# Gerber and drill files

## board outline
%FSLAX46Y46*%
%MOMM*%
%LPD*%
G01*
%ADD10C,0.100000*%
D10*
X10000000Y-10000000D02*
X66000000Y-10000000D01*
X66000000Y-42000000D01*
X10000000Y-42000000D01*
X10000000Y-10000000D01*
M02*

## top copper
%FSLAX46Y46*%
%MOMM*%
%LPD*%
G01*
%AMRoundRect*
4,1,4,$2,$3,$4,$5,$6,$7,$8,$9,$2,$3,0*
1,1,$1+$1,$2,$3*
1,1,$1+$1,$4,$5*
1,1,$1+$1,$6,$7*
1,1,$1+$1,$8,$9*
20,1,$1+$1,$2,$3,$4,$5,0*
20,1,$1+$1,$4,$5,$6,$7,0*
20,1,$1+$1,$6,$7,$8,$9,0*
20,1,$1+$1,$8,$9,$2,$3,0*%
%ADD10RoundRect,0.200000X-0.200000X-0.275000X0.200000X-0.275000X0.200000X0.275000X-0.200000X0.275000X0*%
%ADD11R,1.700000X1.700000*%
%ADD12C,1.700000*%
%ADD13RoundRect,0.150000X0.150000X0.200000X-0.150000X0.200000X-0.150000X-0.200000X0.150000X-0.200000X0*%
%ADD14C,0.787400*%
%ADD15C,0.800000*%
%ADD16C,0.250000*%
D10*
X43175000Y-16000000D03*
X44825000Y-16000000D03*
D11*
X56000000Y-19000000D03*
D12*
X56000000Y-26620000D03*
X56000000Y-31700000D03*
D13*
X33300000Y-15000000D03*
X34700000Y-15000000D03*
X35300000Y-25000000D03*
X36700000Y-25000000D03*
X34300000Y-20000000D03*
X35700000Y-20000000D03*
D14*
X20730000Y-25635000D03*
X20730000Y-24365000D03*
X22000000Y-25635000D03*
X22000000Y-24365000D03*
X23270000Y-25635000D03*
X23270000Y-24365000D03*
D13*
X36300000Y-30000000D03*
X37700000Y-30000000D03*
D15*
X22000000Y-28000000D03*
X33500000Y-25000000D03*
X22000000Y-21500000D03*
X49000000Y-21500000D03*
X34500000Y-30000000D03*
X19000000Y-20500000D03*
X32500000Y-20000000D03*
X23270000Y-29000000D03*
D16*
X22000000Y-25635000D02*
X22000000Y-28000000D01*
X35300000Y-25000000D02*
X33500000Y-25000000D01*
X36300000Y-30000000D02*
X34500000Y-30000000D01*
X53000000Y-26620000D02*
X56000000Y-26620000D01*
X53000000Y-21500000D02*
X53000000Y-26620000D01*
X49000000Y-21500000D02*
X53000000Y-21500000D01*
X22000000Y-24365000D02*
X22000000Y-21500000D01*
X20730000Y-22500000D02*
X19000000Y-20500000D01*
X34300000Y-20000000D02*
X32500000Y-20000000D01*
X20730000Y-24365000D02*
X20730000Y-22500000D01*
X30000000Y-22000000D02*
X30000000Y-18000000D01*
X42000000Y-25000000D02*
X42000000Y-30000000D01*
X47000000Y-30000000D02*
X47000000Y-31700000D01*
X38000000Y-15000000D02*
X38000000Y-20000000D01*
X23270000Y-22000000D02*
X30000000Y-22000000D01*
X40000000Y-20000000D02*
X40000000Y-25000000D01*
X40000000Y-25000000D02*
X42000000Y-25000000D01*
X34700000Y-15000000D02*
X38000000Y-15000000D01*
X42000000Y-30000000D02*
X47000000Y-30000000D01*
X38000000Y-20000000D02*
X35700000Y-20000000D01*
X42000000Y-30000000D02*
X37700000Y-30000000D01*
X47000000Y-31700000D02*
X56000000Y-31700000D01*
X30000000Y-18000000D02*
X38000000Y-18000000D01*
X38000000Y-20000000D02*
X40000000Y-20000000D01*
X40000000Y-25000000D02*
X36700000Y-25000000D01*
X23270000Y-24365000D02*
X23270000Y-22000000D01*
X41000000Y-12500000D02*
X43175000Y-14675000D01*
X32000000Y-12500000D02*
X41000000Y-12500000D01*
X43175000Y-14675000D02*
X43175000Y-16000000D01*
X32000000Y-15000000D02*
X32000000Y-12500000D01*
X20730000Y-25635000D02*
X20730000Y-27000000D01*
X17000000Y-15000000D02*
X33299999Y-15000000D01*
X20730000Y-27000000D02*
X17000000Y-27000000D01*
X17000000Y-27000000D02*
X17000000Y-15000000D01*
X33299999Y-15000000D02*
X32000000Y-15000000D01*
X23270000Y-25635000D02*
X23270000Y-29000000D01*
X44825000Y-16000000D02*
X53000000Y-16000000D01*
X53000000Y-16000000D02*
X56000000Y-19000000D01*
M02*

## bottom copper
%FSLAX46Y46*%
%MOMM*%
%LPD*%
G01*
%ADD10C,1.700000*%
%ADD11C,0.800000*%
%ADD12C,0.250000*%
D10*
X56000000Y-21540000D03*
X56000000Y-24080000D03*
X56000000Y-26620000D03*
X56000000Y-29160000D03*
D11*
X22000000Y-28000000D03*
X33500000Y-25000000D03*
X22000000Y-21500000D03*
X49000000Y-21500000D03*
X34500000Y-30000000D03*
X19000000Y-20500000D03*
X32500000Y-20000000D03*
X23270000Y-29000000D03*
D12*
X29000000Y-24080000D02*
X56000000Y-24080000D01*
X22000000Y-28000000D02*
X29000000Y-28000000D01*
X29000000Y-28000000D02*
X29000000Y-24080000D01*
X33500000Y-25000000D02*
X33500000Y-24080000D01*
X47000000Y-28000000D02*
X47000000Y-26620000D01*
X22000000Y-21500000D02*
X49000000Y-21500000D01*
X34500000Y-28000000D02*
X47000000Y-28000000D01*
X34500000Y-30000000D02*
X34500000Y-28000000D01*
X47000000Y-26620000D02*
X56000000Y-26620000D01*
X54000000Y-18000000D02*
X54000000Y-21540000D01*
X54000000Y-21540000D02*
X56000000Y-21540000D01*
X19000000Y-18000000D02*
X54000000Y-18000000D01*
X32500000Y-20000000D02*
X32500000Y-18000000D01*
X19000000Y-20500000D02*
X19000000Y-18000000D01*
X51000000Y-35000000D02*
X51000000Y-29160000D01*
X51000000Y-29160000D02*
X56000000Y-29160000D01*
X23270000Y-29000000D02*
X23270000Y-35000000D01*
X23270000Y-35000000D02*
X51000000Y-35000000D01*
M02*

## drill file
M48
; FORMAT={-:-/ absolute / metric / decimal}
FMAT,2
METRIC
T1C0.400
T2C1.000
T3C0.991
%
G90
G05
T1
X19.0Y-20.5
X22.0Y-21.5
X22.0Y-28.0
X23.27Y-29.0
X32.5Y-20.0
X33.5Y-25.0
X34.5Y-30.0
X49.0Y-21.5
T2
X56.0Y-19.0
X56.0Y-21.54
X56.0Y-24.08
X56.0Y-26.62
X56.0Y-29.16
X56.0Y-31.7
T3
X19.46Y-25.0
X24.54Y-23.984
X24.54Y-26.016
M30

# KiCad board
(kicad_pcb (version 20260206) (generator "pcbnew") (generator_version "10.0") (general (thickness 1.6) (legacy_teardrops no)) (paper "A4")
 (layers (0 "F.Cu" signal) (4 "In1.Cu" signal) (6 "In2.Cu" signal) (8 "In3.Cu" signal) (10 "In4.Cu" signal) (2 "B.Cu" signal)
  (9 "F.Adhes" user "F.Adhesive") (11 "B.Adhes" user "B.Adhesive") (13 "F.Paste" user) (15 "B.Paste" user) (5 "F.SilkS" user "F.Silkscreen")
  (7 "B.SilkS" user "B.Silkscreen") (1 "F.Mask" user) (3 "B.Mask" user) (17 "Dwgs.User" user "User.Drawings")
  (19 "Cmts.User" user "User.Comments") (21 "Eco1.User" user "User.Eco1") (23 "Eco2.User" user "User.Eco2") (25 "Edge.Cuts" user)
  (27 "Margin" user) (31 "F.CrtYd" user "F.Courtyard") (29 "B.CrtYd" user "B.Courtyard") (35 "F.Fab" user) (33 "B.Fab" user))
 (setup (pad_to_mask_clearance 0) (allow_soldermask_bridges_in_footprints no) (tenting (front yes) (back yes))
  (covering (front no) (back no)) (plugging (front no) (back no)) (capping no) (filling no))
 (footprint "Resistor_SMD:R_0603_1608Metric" (layer "F.Cu") (at 44 16)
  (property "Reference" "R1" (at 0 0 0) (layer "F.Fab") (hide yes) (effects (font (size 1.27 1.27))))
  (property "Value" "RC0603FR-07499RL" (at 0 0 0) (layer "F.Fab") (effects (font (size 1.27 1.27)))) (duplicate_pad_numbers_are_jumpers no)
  (pad "1" smd roundrect (at -0.825 0) (size 0.8 0.95) (layers "F.Cu" "F.Mask" "F.Paste") (roundrect_rratio 0.25) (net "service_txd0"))
  (pad "2" smd roundrect (at 0.825 0) (size 0.8 0.95) (layers "F.Cu" "F.Mask" "F.Paste") (roundrect_rratio 0.25) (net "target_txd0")))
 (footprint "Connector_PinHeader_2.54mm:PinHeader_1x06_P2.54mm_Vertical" (layer "F.Cu") (at 56 19)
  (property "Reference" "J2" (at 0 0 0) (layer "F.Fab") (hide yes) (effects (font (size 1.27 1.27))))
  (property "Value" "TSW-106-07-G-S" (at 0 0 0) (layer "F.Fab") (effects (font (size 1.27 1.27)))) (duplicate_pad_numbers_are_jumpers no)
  (pad "1" thru_hole rect (at 0 0) (size 1.7 1.7) (drill 1) (layers "*.Cu" "*.Mask") (remove_unused_layers yes) (keep_end_layers no)
   (zone_layer_connections) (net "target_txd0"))
  (pad "2" thru_hole circle (at 0 2.54) (size 1.7 1.7) (drill 1) (layers "*.Cu" "*.Mask") (remove_unused_layers yes) (keep_end_layers no)
   (zone_layer_connections) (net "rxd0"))
  (pad "3" thru_hole circle (at 0 5.08) (size 1.7 1.7) (drill 1) (layers "*.Cu" "*.Mask") (remove_unused_layers yes) (keep_end_layers no)
   (zone_layer_connections) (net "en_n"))
  (pad "4" thru_hole circle (at 0 7.62) (size 1.7 1.7) (drill 1) (layers "*.Cu" "*.Mask") (remove_unused_layers yes) (keep_end_layers no)
   (zone_layer_connections) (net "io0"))
  (pad "5" thru_hole circle (at 0 10.16) (size 1.7 1.7) (drill 1) (layers "*.Cu" "*.Mask") (remove_unused_layers yes) (keep_end_layers no)
   (zone_layer_connections) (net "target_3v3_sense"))
  (pad "6" thru_hole circle (at 0 12.7) (size 1.7 1.7) (drill 1) (layers "*.Cu" "*.Mask") (remove_unused_layers yes) (keep_end_layers no)
   (zone_layer_connections) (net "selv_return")))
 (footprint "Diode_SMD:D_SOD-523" (layer "F.Cu") (at 34 15)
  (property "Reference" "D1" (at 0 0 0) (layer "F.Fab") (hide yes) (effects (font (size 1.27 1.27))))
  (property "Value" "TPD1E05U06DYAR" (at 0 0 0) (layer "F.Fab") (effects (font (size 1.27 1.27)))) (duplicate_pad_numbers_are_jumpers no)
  (pad "1" smd roundrect (at -0.7 0 180) (size 0.6 0.7) (layers "F.Cu" "F.Mask" "F.Paste") (roundrect_rratio 0.25) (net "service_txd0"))
  (pad "2" smd roundrect (at 0.7 0 180) (size 0.6 0.7) (layers "F.Cu" "F.Mask" "F.Paste") (roundrect_rratio 0.25) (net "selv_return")))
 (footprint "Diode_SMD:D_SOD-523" (layer "F.Cu") (at 36 25)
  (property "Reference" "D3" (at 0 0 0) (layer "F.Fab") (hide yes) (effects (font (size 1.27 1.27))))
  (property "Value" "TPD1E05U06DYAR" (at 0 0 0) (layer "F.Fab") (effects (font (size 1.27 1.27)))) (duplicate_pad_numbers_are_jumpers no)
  (pad "1" smd roundrect (at -0.7 0 180) (size 0.6 0.7) (layers "F.Cu" "F.Mask" "F.Paste") (roundrect_rratio 0.25) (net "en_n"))
  (pad "2" smd roundrect (at 0.7 0 180) (size 0.6 0.7) (layers "F.Cu" "F.Mask" "F.Paste") (roundrect_rratio 0.25) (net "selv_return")))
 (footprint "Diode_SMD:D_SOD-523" (layer "F.Cu") (at 35 20)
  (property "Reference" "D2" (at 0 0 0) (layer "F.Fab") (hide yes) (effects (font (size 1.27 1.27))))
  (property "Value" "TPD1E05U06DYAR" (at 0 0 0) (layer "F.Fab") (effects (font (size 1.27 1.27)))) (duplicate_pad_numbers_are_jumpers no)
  (pad "1" smd roundrect (at -0.7 0 180) (size 0.6 0.7) (layers "F.Cu" "F.Mask" "F.Paste") (roundrect_rratio 0.25) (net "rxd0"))
  (pad "2" smd roundrect (at 0.7 0 180) (size 0.6 0.7) (layers "F.Cu" "F.Mask" "F.Paste") (roundrect_rratio 0.25) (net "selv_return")))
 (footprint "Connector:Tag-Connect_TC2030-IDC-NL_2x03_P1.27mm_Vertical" (layer "F.Cu") (at 22 25)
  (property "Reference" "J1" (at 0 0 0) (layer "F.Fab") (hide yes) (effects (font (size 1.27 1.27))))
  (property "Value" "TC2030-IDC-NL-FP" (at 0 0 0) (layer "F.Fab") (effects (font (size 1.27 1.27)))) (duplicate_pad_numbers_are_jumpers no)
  (pad "" np_thru_hole circle (at -2.54 0) (size 0.9906 0.9906) (drill 0.9906) (layers "*.Cu" "*.Mask"))
  (pad "" np_thru_hole circle (at 2.54 -1.016) (size 0.9906 0.9906) (drill 0.9906) (layers "*.Cu" "*.Mask"))
  (pad "" np_thru_hole circle (at 2.54 1.016) (size 0.9906 0.9906) (drill 0.9906) (layers "*.Cu" "*.Mask"))
  (pad "1" connect circle (at -1.27 0.635) (size 0.7874 0.7874) (layers "F.Cu" "F.Mask") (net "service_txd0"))
  (pad "2" connect circle (at -1.27 -0.635) (size 0.7874 0.7874) (layers "F.Cu" "F.Mask") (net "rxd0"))
  (pad "3" connect circle (at 0 0.635) (size 0.7874 0.7874) (layers "F.Cu" "F.Mask") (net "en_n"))
  (pad "4" connect circle (at 0 -0.635) (size 0.7874 0.7874) (layers "F.Cu" "F.Mask") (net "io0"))
  (pad "5" connect circle (at 1.27 0.635) (size 0.7874 0.7874) (layers "F.Cu" "F.Mask") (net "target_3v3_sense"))
  (pad "6" connect circle (at 1.27 -0.635) (size 0.7874 0.7874) (layers "F.Cu" "F.Mask") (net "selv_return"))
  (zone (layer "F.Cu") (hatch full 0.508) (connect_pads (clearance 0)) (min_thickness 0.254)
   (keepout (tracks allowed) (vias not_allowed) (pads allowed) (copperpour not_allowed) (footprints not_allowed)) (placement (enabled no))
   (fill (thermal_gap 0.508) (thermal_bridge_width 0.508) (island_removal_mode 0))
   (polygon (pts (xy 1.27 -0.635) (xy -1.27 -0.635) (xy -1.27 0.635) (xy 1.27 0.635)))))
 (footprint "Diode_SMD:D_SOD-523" (layer "F.Cu") (at 37 30)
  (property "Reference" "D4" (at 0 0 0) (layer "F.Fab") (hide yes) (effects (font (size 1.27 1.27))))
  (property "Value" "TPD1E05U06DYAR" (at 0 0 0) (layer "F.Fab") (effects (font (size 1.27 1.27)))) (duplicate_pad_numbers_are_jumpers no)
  (pad "1" smd roundrect (at -0.7 0 180) (size 0.6 0.7) (layers "F.Cu" "F.Mask" "F.Paste") (roundrect_rratio 0.25) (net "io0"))
  (pad "2" smd roundrect (at 0.7 0 180) (size 0.6 0.7) (layers "F.Cu" "F.Mask" "F.Paste") (roundrect_rratio 0.25) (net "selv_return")))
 (gr_poly (pts (xy 10 10) (xy 66 10) (xy 66 42) (xy 10 42)) (stroke (width 0.1) (type solid)) (fill no) (layer "Edge.Cuts"))
 (segment (start 22 25.635) (end 22 28) (width 0.25) (layer "F.Cu") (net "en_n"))
 (segment (start 35.3 25) (end 33.5 25) (width 0.25) (layer "F.Cu") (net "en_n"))
 (via (at 22 28) (size 0.8) (drill 0.4) (layers "F.Cu" "B.Cu") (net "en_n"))
 (via (at 33.5 25) (size 0.8) (drill 0.4) (layers "F.Cu" "B.Cu") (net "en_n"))
 (segment (start 29 24.08) (end 56 24.08) (width 0.25) (layer "B.Cu") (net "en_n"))
 (segment (start 22 28) (end 29 28) (width 0.25) (layer "B.Cu") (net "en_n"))
 (segment (start 29 28) (end 29 24.08) (width 0.25) (layer "B.Cu") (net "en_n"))
 (segment (start 33.5 25) (end 33.5 24.08) (width 0.25) (layer "B.Cu") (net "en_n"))
 (segment (start 36.3 30) (end 34.5 30) (width 0.25) (layer "F.Cu") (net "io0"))
 (segment (start 53 26.62) (end 56 26.62) (width 0.25) (layer "F.Cu") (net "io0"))
 (segment (start 53 21.5) (end 53 26.62) (width 0.25) (layer "F.Cu") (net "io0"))
 (segment (start 49 21.5) (end 53 21.5) (width 0.25) (layer "F.Cu") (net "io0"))
 (segment (start 22 24.365) (end 22 21.5) (width 0.25) (layer "F.Cu") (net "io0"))
 (via (at 22 21.5) (size 0.8) (drill 0.4) (layers "F.Cu" "B.Cu") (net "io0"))
 (via (at 49 21.5) (size 0.8) (drill 0.4) (layers "F.Cu" "B.Cu") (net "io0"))
 (via (at 34.5 30) (size 0.8) (drill 0.4) (layers "F.Cu" "B.Cu") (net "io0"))
 (segment (start 47 28) (end 47 26.62) (width 0.25) (layer "B.Cu") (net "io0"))
 (segment (start 22 21.5) (end 49 21.5) (width 0.25) (layer "B.Cu") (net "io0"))
 (segment (start 34.5 28) (end 47 28) (width 0.25) (layer "B.Cu") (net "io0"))
 (segment (start 34.5 30) (end 34.5 28) (width 0.25) (layer "B.Cu") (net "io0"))
 (segment (start 47 26.62) (end 56 26.62) (width 0.25) (layer "B.Cu") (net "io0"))
 (segment (start 20.73 22.5) (end 19 20.5) (width 0.25) (layer "F.Cu") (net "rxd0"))
 (segment (start 34.3 20) (end 32.5 20) (width 0.25) (layer "F.Cu") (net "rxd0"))
 (segment (start 20.73 24.365) (end 20.73 22.5) (width 0.25) (layer "F.Cu") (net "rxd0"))
 (via (at 19 20.5) (size 0.8) (drill 0.4) (layers "F.Cu" "B.Cu") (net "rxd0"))
 (via (at 32.5 20) (size 0.8) (drill 0.4) (layers "F.Cu" "B.Cu") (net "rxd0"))
 (segment (start 54 18) (end 54 21.54) (width 0.25) (layer "B.Cu") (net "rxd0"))
 (segment (start 54 21.54) (end 56 21.54) (width 0.25) (layer "B.Cu") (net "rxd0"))
 (segment (start 19 18) (end 54 18) (width 0.25) (layer "B.Cu") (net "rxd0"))
 (segment (start 32.5 20) (end 32.5 18) (width 0.25) (layer "B.Cu") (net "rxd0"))
 (segment (start 19 20.5) (end 19 18) (width 0.25) (layer "B.Cu") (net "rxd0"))
 (segment (start 30 22) (end 30 18) (width 0.25) (layer "F.Cu") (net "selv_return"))
 (segment (start 42 25) (end 42 30) (width 0.25) (layer "F.Cu") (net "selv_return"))
 (segment (start 47 30) (end 47 31.7) (width 0.25) (layer "F.Cu") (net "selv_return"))
 (segment (start 38 15) (end 38 20) (width 0.25) (layer "F.Cu") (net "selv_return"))
 (segment (start 23.27 22) (end 30 22) (width 0.25) (layer "F.Cu") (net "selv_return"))
 (segment (start 40 20) (end 40 25) (width 0.25) (layer "F.Cu") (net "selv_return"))
 (segment (start 40 25) (end 42 25) (width 0.25) (layer "F.Cu") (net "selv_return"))
 (segment (start 34.7 15) (end 38 15) (width 0.25) (layer "F.Cu") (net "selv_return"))
 (segment (start 42 30) (end 47 30) (width 0.25) (layer "F.Cu") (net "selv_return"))
 (segment (start 38 20) (end 35.7 20) (width 0.25) (layer "F.Cu") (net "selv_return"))
 (segment (start 42 30) (end 37.7 30) (width 0.25) (layer "F.Cu") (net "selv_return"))
 (segment (start 47 31.7) (end 56 31.7) (width 0.25) (layer "F.Cu") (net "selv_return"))
 (segment (start 30 18) (end 38 18) (width 0.25) (layer "F.Cu") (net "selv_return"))
 (segment (start 38 20) (end 40 20) (width 0.25) (layer "F.Cu") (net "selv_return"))
 (segment (start 40 25) (end 36.7 25) (width 0.25) (layer "F.Cu") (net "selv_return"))
 (segment (start 23.27 24.365) (end 23.27 22) (width 0.25) (layer "F.Cu") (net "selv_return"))
 (segment (start 41 12.5) (end 43.175 14.675) (width 0.25) (layer "F.Cu") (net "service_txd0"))
 (segment (start 32 12.5) (end 41 12.5) (width 0.25) (layer "F.Cu") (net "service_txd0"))
 (segment (start 43.175 14.675) (end 43.175 16) (width 0.25) (layer "F.Cu") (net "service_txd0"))
 (segment (start 32 15) (end 32 12.5) (width 0.25) (layer "F.Cu") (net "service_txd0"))
 (segment (start 20.73 25.635) (end 20.73 27) (width 0.25) (layer "F.Cu") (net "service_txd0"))
 (segment (start 17 15) (end 33.299999 15) (width 0.25) (layer "F.Cu") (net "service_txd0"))
 (segment (start 20.73 27) (end 17 27) (width 0.25) (layer "F.Cu") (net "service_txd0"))
 (segment (start 17 27) (end 17 15) (width 0.25) (layer "F.Cu") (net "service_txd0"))
 (segment (start 33.299999 15) (end 32 15) (width 0.25) (layer "F.Cu") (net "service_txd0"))
 (segment (start 23.27 25.635) (end 23.27 29) (width 0.25) (layer "F.Cu") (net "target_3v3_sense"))
 (via (at 23.27 29) (size 0.8) (drill 0.4) (layers "F.Cu" "B.Cu") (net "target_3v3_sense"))
 (segment (start 51 35) (end 51 29.16) (width 0.25) (layer "B.Cu") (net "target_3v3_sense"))
 (segment (start 51 29.16) (end 56 29.16) (width 0.25) (layer "B.Cu") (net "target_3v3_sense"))
 (segment (start 23.27 29) (end 23.27 35) (width 0.25) (layer "B.Cu") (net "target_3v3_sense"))
 (segment (start 23.27 35) (end 51 35) (width 0.25) (layer "B.Cu") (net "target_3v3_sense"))
 (segment (start 44.825 16) (end 53 16) (width 0.25) (layer "F.Cu") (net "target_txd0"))
 (segment (start 53 16) (end 56 19) (width 0.25) (layer "F.Cu") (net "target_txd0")))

